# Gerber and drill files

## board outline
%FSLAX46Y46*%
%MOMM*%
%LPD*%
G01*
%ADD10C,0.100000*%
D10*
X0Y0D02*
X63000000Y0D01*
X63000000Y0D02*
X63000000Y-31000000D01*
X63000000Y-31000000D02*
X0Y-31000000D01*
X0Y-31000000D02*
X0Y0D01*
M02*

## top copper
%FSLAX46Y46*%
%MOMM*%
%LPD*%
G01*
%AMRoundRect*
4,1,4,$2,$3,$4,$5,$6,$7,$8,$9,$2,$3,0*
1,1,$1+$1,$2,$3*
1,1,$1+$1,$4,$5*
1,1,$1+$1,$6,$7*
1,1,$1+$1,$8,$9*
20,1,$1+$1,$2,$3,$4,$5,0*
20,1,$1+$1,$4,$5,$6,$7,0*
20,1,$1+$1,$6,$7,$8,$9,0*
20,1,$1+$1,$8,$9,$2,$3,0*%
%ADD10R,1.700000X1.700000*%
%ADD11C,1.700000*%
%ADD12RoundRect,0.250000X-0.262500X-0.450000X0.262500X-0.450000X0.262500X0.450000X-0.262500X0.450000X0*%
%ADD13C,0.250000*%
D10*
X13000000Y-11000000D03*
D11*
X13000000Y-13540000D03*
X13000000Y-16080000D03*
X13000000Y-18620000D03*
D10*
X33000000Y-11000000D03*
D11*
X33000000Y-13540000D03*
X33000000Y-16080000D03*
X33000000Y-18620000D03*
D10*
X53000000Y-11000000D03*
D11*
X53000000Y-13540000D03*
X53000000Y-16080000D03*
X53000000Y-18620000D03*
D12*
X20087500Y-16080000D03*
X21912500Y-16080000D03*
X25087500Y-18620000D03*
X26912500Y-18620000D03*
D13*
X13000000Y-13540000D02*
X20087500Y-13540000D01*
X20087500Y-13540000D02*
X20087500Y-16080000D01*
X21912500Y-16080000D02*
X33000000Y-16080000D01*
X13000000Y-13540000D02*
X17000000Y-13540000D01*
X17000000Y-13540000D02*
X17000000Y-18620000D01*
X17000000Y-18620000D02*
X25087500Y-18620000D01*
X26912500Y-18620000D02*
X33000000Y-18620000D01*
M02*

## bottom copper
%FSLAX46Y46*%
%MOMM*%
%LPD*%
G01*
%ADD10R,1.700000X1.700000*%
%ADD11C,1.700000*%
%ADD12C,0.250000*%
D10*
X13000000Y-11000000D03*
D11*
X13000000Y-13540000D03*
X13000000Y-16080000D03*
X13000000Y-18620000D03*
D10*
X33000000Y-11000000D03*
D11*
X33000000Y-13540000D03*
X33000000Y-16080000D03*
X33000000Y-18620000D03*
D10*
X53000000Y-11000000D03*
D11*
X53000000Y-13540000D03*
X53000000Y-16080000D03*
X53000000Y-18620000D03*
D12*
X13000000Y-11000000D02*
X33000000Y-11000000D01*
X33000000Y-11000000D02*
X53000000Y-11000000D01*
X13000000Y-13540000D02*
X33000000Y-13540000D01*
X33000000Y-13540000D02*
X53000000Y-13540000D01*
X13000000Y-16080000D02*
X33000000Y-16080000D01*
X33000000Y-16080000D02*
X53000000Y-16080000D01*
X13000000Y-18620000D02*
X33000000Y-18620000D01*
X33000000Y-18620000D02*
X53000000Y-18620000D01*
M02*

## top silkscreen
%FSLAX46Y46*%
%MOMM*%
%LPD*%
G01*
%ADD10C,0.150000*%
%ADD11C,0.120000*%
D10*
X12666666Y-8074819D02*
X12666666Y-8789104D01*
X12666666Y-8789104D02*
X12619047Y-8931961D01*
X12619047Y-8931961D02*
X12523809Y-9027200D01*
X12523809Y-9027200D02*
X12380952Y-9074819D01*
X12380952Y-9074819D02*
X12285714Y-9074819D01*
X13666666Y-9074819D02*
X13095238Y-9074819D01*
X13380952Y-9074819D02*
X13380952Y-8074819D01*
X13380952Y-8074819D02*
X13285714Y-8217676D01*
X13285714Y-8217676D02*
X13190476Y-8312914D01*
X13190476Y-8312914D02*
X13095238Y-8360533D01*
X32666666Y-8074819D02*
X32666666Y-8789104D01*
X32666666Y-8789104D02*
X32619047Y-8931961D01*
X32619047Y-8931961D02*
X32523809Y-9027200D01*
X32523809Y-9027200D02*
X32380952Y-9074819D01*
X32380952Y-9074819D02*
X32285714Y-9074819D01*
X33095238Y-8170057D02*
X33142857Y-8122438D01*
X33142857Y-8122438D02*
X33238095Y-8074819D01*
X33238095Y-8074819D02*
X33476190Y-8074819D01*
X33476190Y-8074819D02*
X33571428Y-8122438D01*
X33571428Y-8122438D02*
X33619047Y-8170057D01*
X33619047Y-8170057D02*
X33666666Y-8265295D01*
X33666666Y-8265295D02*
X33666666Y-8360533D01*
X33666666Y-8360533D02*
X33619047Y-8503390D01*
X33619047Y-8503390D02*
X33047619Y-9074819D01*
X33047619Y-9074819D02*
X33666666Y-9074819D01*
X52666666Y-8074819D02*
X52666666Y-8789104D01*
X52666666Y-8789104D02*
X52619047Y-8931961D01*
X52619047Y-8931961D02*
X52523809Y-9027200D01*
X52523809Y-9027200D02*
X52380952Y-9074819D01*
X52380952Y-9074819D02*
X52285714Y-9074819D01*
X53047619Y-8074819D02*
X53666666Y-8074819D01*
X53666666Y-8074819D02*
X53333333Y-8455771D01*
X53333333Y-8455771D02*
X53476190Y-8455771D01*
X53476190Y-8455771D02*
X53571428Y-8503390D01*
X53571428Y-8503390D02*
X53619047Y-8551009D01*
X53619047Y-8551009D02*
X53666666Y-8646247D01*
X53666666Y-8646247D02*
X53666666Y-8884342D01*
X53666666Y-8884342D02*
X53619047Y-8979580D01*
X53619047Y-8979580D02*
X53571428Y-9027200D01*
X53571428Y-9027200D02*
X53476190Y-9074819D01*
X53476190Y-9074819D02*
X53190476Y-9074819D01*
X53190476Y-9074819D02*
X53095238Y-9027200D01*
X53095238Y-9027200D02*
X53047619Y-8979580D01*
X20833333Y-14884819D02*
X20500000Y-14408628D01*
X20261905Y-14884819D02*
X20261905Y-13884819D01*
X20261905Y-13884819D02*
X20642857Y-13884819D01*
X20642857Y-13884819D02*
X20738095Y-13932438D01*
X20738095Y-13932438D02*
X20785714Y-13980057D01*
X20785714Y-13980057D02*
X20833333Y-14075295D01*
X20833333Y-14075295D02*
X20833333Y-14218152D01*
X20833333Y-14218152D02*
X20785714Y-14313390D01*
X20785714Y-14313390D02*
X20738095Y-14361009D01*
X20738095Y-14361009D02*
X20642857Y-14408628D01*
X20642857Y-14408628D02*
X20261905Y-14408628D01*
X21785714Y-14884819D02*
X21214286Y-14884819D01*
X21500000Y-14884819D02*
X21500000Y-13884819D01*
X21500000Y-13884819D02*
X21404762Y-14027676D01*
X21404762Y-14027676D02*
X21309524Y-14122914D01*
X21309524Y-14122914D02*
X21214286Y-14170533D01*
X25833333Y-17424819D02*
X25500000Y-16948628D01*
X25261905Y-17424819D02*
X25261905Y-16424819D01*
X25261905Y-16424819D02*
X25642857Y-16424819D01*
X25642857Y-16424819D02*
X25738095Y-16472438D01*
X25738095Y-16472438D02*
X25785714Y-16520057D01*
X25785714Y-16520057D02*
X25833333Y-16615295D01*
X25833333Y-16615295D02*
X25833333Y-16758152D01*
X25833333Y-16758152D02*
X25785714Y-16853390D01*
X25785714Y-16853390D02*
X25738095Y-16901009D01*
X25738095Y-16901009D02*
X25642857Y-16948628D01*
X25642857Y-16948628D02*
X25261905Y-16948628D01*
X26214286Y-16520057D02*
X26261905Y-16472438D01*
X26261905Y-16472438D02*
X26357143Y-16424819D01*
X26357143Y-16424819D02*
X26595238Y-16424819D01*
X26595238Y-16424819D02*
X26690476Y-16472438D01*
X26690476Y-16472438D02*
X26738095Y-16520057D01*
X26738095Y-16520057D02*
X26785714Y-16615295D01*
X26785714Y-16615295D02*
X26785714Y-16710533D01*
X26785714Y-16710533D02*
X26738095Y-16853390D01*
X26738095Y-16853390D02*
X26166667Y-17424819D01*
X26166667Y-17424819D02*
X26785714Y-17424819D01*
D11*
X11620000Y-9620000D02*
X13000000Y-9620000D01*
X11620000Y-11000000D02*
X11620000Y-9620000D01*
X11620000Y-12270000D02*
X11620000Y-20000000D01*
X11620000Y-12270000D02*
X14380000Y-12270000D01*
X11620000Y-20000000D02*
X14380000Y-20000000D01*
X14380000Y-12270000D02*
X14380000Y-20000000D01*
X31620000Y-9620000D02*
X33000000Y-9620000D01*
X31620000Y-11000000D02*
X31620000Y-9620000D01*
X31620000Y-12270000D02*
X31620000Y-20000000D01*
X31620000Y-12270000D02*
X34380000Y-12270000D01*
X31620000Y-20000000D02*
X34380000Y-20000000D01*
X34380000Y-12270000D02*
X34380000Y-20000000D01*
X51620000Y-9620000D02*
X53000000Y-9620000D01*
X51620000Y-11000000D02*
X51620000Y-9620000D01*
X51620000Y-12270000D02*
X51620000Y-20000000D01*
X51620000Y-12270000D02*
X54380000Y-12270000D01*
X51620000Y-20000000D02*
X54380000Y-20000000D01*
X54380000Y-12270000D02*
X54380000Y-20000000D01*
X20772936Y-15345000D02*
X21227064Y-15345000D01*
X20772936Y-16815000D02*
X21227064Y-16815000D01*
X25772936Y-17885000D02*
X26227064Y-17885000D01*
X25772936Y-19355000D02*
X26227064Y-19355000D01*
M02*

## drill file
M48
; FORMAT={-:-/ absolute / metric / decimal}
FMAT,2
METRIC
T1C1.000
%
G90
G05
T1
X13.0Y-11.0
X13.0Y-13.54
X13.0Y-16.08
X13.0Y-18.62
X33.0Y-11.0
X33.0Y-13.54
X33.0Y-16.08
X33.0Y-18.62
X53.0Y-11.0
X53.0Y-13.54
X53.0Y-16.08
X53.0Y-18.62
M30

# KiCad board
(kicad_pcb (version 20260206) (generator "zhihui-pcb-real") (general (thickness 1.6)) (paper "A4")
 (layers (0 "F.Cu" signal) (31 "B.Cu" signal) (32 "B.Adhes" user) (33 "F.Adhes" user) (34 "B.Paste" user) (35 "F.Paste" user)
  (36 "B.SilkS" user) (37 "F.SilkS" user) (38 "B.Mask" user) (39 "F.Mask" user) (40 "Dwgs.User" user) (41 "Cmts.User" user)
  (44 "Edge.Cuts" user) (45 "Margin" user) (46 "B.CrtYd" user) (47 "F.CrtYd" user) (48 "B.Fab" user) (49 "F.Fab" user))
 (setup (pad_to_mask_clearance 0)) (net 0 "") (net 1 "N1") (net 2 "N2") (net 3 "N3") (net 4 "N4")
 (gr_line (start 0 0) (end 63 0) (stroke (width 0.1) (type default)) (layer "Edge.Cuts"))
 (gr_line (start 63 0) (end 63 31) (stroke (width 0.1) (type default)) (layer "Edge.Cuts"))
 (gr_line (start 63 31) (end 0 31) (stroke (width 0.1) (type default)) (layer "Edge.Cuts"))
 (gr_line (start 0 31) (end 0 0) (stroke (width 0.1) (type default)) (layer "Edge.Cuts"))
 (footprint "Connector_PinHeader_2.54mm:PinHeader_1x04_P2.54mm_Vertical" (layer "F.Cu")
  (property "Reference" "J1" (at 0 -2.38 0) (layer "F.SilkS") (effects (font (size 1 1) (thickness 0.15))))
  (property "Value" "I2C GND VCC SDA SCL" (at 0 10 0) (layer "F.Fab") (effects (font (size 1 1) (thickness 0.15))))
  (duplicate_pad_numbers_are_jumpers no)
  (fp_line (start -1.38 -1.38) (end 0 -1.38) (stroke (width 0.12) (type solid)) (layer "F.SilkS"))
  (fp_line (start -1.38 0) (end -1.38 -1.38) (stroke (width 0.12) (type solid)) (layer "F.SilkS"))
  (fp_line (start -1.38 1.27) (end -1.38 9) (stroke (width 0.12) (type solid)) (layer "F.SilkS"))
  (fp_line (start -1.38 1.27) (end 1.38 1.27) (stroke (width 0.12) (type solid)) (layer "F.SilkS"))
  (fp_line (start -1.38 9) (end 1.38 9) (stroke (width 0.12) (type solid)) (layer "F.SilkS"))
  (fp_line (start 1.38 1.27) (end 1.38 9) (stroke (width 0.12) (type solid)) (layer "F.SilkS"))
  (pad "1" thru_hole rect (at 0 0) (size 1.7 1.7) (drill 1) (layers "*.Cu" "*.Mask") (remove_unused_layers no) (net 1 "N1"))
  (pad "2" thru_hole circle (at 0 2.54) (size 1.7 1.7) (drill 1) (layers "*.Cu" "*.Mask") (remove_unused_layers no) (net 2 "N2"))
  (pad "3" thru_hole circle (at 0 5.08) (size 1.7 1.7) (drill 1) (layers "*.Cu" "*.Mask") (remove_unused_layers no) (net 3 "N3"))
  (pad "4" thru_hole circle (at 0 7.62) (size 1.7 1.7) (drill 1) (layers "*.Cu" "*.Mask") (remove_unused_layers no) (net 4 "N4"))
  (at 13 11 0))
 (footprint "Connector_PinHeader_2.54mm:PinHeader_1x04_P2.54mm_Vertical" (layer "F.Cu")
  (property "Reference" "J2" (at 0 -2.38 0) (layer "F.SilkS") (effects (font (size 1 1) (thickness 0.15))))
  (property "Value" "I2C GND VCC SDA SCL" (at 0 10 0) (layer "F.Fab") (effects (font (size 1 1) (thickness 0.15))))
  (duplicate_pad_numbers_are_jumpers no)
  (fp_line (start -1.38 -1.38) (end 0 -1.38) (stroke (width 0.12) (type solid)) (layer "F.SilkS"))
  (fp_line (start -1.38 0) (end -1.38 -1.38) (stroke (width 0.12) (type solid)) (layer "F.SilkS"))
  (fp_line (start -1.38 1.27) (end -1.38 9) (stroke (width 0.12) (type solid)) (layer "F.SilkS"))
  (fp_line (start -1.38 1.27) (end 1.38 1.27) (stroke (width 0.12) (type solid)) (layer "F.SilkS"))
  (fp_line (start -1.38 9) (end 1.38 9) (stroke (width 0.12) (type solid)) (layer "F.SilkS"))
  (fp_line (start 1.38 1.27) (end 1.38 9) (stroke (width 0.12) (type solid)) (layer "F.SilkS"))
  (pad "1" thru_hole rect (at 0 0) (size 1.7 1.7) (drill 1) (layers "*.Cu" "*.Mask") (remove_unused_layers no) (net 1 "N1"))
  (pad "2" thru_hole circle (at 0 2.54) (size 1.7 1.7) (drill 1) (layers "*.Cu" "*.Mask") (remove_unused_layers no) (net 2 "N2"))
  (pad "3" thru_hole circle (at 0 5.08) (size 1.7 1.7) (drill 1) (layers "*.Cu" "*.Mask") (remove_unused_layers no) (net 3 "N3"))
  (pad "4" thru_hole circle (at 0 7.62) (size 1.7 1.7) (drill 1) (layers "*.Cu" "*.Mask") (remove_unused_layers no) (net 4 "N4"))
  (at 33 11 0))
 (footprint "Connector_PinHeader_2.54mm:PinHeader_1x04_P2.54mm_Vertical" (layer "F.Cu")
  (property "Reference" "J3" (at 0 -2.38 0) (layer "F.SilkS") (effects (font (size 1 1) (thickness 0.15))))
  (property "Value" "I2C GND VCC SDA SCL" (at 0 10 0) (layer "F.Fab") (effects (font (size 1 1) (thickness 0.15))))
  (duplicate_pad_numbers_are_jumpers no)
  (fp_line (start -1.38 -1.38) (end 0 -1.38) (stroke (width 0.12) (type solid)) (layer "F.SilkS"))
  (fp_line (start -1.38 0) (end -1.38 -1.38) (stroke (width 0.12) (type solid)) (layer "F.SilkS"))
  (fp_line (start -1.38 1.27) (end -1.38 9) (stroke (width 0.12) (type solid)) (layer "F.SilkS"))
  (fp_line (start -1.38 1.27) (end 1.38 1.27) (stroke (width 0.12) (type solid)) (layer "F.SilkS"))
  (fp_line (start -1.38 9) (end 1.38 9) (stroke (width 0.12) (type solid)) (layer "F.SilkS"))
  (fp_line (start 1.38 1.27) (end 1.38 9) (stroke (width 0.12) (type solid)) (layer "F.SilkS"))
  (pad "1" thru_hole rect (at 0 0) (size 1.7 1.7) (drill 1) (layers "*.Cu" "*.Mask") (remove_unused_layers no) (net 1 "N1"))
  (pad "2" thru_hole circle (at 0 2.54) (size 1.7 1.7) (drill 1) (layers "*.Cu" "*.Mask") (remove_unused_layers no) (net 2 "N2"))
  (pad "3" thru_hole circle (at 0 5.08) (size 1.7 1.7) (drill 1) (layers "*.Cu" "*.Mask") (remove_unused_layers no) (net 3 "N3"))
  (pad "4" thru_hole circle (at 0 7.62) (size 1.7 1.7) (drill 1) (layers "*.Cu" "*.Mask") (remove_unused_layers no) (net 4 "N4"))
  (at 53 11 0))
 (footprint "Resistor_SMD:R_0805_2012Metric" (layer "F.Cu")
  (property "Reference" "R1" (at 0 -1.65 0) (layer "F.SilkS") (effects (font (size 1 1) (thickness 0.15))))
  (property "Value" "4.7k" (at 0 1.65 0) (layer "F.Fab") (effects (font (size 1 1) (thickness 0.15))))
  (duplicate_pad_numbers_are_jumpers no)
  (fp_line (start -0.227064 -0.735) (end 0.227064 -0.735) (stroke (width 0.12) (type solid)) (layer "F.SilkS"))
  (fp_line (start -0.227064 0.735) (end 0.227064 0.735) (stroke (width 0.12) (type solid)) (layer "F.SilkS"))
  (pad "1" smd roundrect (at -0.9125 0) (size 1.025 1.4) (layers "F.Cu" "F.Mask" "F.Paste") (roundrect_rratio 0.243902) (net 2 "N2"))
  (pad "2" smd roundrect (at 0.9125 0) (size 1.025 1.4) (layers "F.Cu" "F.Mask" "F.Paste") (roundrect_rratio 0.243902) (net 3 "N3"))
  (at 21 16.08 0))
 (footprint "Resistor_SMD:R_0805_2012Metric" (layer "F.Cu")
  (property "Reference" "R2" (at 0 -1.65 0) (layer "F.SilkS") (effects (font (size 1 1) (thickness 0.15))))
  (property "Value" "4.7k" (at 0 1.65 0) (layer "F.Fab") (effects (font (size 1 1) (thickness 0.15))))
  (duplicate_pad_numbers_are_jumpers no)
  (fp_line (start -0.227064 -0.735) (end 0.227064 -0.735) (stroke (width 0.12) (type solid)) (layer "F.SilkS"))
  (fp_line (start -0.227064 0.735) (end 0.227064 0.735) (stroke (width 0.12) (type solid)) (layer "F.SilkS"))
  (pad "1" smd roundrect (at -0.9125 0) (size 1.025 1.4) (layers "F.Cu" "F.Mask" "F.Paste") (roundrect_rratio 0.243902) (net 2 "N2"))
  (pad "2" smd roundrect (at 0.9125 0) (size 1.025 1.4) (layers "F.Cu" "F.Mask" "F.Paste") (roundrect_rratio 0.243902) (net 4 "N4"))
  (at 26 18.62 0))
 (segment (start 13 11) (end 33 11) (width 0.25) (layer "B.Cu") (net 1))
 (segment (start 33 11) (end 53 11) (width 0.25) (layer "B.Cu") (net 1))
 (segment (start 13 13.54) (end 33 13.54) (width 0.25) (layer "B.Cu") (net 2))
 (segment (start 33 13.54) (end 53 13.54) (width 0.25) (layer "B.Cu") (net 2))
 (segment (start 13 16.08) (end 33 16.08) (width 0.25) (layer "B.Cu") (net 3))
 (segment (start 33 16.08) (end 53 16.08) (width 0.25) (layer "B.Cu") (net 3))
 (segment (start 13 18.62) (end 33 18.62) (width 0.25) (layer "B.Cu") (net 4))
 (segment (start 33 18.62) (end 53 18.62) (width 0.25) (layer "B.Cu") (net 4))
 (segment (start 13 13.54) (end 20.0875 13.54) (width 0.25) (layer "F.Cu") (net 2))
 (segment (start 20.0875 13.54) (end 20.0875 16.08) (width 0.25) (layer "F.Cu") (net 2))
 (segment (start 21.9125 16.08) (end 33 16.08) (width 0.25) (layer "F.Cu") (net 3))
 (segment (start 13 13.54) (end 17 13.54) (width 0.25) (layer "F.Cu") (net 2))
 (segment (start 17 13.54) (end 17 18.62) (width 0.25) (layer "F.Cu") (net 2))
 (segment (start 17 18.62) (end 25.0875 18.62) (width 0.25) (layer "F.Cu") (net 2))
 (segment (start 26.9125 18.62) (end 33 18.62) (width 0.25) (layer "F.Cu") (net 4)))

